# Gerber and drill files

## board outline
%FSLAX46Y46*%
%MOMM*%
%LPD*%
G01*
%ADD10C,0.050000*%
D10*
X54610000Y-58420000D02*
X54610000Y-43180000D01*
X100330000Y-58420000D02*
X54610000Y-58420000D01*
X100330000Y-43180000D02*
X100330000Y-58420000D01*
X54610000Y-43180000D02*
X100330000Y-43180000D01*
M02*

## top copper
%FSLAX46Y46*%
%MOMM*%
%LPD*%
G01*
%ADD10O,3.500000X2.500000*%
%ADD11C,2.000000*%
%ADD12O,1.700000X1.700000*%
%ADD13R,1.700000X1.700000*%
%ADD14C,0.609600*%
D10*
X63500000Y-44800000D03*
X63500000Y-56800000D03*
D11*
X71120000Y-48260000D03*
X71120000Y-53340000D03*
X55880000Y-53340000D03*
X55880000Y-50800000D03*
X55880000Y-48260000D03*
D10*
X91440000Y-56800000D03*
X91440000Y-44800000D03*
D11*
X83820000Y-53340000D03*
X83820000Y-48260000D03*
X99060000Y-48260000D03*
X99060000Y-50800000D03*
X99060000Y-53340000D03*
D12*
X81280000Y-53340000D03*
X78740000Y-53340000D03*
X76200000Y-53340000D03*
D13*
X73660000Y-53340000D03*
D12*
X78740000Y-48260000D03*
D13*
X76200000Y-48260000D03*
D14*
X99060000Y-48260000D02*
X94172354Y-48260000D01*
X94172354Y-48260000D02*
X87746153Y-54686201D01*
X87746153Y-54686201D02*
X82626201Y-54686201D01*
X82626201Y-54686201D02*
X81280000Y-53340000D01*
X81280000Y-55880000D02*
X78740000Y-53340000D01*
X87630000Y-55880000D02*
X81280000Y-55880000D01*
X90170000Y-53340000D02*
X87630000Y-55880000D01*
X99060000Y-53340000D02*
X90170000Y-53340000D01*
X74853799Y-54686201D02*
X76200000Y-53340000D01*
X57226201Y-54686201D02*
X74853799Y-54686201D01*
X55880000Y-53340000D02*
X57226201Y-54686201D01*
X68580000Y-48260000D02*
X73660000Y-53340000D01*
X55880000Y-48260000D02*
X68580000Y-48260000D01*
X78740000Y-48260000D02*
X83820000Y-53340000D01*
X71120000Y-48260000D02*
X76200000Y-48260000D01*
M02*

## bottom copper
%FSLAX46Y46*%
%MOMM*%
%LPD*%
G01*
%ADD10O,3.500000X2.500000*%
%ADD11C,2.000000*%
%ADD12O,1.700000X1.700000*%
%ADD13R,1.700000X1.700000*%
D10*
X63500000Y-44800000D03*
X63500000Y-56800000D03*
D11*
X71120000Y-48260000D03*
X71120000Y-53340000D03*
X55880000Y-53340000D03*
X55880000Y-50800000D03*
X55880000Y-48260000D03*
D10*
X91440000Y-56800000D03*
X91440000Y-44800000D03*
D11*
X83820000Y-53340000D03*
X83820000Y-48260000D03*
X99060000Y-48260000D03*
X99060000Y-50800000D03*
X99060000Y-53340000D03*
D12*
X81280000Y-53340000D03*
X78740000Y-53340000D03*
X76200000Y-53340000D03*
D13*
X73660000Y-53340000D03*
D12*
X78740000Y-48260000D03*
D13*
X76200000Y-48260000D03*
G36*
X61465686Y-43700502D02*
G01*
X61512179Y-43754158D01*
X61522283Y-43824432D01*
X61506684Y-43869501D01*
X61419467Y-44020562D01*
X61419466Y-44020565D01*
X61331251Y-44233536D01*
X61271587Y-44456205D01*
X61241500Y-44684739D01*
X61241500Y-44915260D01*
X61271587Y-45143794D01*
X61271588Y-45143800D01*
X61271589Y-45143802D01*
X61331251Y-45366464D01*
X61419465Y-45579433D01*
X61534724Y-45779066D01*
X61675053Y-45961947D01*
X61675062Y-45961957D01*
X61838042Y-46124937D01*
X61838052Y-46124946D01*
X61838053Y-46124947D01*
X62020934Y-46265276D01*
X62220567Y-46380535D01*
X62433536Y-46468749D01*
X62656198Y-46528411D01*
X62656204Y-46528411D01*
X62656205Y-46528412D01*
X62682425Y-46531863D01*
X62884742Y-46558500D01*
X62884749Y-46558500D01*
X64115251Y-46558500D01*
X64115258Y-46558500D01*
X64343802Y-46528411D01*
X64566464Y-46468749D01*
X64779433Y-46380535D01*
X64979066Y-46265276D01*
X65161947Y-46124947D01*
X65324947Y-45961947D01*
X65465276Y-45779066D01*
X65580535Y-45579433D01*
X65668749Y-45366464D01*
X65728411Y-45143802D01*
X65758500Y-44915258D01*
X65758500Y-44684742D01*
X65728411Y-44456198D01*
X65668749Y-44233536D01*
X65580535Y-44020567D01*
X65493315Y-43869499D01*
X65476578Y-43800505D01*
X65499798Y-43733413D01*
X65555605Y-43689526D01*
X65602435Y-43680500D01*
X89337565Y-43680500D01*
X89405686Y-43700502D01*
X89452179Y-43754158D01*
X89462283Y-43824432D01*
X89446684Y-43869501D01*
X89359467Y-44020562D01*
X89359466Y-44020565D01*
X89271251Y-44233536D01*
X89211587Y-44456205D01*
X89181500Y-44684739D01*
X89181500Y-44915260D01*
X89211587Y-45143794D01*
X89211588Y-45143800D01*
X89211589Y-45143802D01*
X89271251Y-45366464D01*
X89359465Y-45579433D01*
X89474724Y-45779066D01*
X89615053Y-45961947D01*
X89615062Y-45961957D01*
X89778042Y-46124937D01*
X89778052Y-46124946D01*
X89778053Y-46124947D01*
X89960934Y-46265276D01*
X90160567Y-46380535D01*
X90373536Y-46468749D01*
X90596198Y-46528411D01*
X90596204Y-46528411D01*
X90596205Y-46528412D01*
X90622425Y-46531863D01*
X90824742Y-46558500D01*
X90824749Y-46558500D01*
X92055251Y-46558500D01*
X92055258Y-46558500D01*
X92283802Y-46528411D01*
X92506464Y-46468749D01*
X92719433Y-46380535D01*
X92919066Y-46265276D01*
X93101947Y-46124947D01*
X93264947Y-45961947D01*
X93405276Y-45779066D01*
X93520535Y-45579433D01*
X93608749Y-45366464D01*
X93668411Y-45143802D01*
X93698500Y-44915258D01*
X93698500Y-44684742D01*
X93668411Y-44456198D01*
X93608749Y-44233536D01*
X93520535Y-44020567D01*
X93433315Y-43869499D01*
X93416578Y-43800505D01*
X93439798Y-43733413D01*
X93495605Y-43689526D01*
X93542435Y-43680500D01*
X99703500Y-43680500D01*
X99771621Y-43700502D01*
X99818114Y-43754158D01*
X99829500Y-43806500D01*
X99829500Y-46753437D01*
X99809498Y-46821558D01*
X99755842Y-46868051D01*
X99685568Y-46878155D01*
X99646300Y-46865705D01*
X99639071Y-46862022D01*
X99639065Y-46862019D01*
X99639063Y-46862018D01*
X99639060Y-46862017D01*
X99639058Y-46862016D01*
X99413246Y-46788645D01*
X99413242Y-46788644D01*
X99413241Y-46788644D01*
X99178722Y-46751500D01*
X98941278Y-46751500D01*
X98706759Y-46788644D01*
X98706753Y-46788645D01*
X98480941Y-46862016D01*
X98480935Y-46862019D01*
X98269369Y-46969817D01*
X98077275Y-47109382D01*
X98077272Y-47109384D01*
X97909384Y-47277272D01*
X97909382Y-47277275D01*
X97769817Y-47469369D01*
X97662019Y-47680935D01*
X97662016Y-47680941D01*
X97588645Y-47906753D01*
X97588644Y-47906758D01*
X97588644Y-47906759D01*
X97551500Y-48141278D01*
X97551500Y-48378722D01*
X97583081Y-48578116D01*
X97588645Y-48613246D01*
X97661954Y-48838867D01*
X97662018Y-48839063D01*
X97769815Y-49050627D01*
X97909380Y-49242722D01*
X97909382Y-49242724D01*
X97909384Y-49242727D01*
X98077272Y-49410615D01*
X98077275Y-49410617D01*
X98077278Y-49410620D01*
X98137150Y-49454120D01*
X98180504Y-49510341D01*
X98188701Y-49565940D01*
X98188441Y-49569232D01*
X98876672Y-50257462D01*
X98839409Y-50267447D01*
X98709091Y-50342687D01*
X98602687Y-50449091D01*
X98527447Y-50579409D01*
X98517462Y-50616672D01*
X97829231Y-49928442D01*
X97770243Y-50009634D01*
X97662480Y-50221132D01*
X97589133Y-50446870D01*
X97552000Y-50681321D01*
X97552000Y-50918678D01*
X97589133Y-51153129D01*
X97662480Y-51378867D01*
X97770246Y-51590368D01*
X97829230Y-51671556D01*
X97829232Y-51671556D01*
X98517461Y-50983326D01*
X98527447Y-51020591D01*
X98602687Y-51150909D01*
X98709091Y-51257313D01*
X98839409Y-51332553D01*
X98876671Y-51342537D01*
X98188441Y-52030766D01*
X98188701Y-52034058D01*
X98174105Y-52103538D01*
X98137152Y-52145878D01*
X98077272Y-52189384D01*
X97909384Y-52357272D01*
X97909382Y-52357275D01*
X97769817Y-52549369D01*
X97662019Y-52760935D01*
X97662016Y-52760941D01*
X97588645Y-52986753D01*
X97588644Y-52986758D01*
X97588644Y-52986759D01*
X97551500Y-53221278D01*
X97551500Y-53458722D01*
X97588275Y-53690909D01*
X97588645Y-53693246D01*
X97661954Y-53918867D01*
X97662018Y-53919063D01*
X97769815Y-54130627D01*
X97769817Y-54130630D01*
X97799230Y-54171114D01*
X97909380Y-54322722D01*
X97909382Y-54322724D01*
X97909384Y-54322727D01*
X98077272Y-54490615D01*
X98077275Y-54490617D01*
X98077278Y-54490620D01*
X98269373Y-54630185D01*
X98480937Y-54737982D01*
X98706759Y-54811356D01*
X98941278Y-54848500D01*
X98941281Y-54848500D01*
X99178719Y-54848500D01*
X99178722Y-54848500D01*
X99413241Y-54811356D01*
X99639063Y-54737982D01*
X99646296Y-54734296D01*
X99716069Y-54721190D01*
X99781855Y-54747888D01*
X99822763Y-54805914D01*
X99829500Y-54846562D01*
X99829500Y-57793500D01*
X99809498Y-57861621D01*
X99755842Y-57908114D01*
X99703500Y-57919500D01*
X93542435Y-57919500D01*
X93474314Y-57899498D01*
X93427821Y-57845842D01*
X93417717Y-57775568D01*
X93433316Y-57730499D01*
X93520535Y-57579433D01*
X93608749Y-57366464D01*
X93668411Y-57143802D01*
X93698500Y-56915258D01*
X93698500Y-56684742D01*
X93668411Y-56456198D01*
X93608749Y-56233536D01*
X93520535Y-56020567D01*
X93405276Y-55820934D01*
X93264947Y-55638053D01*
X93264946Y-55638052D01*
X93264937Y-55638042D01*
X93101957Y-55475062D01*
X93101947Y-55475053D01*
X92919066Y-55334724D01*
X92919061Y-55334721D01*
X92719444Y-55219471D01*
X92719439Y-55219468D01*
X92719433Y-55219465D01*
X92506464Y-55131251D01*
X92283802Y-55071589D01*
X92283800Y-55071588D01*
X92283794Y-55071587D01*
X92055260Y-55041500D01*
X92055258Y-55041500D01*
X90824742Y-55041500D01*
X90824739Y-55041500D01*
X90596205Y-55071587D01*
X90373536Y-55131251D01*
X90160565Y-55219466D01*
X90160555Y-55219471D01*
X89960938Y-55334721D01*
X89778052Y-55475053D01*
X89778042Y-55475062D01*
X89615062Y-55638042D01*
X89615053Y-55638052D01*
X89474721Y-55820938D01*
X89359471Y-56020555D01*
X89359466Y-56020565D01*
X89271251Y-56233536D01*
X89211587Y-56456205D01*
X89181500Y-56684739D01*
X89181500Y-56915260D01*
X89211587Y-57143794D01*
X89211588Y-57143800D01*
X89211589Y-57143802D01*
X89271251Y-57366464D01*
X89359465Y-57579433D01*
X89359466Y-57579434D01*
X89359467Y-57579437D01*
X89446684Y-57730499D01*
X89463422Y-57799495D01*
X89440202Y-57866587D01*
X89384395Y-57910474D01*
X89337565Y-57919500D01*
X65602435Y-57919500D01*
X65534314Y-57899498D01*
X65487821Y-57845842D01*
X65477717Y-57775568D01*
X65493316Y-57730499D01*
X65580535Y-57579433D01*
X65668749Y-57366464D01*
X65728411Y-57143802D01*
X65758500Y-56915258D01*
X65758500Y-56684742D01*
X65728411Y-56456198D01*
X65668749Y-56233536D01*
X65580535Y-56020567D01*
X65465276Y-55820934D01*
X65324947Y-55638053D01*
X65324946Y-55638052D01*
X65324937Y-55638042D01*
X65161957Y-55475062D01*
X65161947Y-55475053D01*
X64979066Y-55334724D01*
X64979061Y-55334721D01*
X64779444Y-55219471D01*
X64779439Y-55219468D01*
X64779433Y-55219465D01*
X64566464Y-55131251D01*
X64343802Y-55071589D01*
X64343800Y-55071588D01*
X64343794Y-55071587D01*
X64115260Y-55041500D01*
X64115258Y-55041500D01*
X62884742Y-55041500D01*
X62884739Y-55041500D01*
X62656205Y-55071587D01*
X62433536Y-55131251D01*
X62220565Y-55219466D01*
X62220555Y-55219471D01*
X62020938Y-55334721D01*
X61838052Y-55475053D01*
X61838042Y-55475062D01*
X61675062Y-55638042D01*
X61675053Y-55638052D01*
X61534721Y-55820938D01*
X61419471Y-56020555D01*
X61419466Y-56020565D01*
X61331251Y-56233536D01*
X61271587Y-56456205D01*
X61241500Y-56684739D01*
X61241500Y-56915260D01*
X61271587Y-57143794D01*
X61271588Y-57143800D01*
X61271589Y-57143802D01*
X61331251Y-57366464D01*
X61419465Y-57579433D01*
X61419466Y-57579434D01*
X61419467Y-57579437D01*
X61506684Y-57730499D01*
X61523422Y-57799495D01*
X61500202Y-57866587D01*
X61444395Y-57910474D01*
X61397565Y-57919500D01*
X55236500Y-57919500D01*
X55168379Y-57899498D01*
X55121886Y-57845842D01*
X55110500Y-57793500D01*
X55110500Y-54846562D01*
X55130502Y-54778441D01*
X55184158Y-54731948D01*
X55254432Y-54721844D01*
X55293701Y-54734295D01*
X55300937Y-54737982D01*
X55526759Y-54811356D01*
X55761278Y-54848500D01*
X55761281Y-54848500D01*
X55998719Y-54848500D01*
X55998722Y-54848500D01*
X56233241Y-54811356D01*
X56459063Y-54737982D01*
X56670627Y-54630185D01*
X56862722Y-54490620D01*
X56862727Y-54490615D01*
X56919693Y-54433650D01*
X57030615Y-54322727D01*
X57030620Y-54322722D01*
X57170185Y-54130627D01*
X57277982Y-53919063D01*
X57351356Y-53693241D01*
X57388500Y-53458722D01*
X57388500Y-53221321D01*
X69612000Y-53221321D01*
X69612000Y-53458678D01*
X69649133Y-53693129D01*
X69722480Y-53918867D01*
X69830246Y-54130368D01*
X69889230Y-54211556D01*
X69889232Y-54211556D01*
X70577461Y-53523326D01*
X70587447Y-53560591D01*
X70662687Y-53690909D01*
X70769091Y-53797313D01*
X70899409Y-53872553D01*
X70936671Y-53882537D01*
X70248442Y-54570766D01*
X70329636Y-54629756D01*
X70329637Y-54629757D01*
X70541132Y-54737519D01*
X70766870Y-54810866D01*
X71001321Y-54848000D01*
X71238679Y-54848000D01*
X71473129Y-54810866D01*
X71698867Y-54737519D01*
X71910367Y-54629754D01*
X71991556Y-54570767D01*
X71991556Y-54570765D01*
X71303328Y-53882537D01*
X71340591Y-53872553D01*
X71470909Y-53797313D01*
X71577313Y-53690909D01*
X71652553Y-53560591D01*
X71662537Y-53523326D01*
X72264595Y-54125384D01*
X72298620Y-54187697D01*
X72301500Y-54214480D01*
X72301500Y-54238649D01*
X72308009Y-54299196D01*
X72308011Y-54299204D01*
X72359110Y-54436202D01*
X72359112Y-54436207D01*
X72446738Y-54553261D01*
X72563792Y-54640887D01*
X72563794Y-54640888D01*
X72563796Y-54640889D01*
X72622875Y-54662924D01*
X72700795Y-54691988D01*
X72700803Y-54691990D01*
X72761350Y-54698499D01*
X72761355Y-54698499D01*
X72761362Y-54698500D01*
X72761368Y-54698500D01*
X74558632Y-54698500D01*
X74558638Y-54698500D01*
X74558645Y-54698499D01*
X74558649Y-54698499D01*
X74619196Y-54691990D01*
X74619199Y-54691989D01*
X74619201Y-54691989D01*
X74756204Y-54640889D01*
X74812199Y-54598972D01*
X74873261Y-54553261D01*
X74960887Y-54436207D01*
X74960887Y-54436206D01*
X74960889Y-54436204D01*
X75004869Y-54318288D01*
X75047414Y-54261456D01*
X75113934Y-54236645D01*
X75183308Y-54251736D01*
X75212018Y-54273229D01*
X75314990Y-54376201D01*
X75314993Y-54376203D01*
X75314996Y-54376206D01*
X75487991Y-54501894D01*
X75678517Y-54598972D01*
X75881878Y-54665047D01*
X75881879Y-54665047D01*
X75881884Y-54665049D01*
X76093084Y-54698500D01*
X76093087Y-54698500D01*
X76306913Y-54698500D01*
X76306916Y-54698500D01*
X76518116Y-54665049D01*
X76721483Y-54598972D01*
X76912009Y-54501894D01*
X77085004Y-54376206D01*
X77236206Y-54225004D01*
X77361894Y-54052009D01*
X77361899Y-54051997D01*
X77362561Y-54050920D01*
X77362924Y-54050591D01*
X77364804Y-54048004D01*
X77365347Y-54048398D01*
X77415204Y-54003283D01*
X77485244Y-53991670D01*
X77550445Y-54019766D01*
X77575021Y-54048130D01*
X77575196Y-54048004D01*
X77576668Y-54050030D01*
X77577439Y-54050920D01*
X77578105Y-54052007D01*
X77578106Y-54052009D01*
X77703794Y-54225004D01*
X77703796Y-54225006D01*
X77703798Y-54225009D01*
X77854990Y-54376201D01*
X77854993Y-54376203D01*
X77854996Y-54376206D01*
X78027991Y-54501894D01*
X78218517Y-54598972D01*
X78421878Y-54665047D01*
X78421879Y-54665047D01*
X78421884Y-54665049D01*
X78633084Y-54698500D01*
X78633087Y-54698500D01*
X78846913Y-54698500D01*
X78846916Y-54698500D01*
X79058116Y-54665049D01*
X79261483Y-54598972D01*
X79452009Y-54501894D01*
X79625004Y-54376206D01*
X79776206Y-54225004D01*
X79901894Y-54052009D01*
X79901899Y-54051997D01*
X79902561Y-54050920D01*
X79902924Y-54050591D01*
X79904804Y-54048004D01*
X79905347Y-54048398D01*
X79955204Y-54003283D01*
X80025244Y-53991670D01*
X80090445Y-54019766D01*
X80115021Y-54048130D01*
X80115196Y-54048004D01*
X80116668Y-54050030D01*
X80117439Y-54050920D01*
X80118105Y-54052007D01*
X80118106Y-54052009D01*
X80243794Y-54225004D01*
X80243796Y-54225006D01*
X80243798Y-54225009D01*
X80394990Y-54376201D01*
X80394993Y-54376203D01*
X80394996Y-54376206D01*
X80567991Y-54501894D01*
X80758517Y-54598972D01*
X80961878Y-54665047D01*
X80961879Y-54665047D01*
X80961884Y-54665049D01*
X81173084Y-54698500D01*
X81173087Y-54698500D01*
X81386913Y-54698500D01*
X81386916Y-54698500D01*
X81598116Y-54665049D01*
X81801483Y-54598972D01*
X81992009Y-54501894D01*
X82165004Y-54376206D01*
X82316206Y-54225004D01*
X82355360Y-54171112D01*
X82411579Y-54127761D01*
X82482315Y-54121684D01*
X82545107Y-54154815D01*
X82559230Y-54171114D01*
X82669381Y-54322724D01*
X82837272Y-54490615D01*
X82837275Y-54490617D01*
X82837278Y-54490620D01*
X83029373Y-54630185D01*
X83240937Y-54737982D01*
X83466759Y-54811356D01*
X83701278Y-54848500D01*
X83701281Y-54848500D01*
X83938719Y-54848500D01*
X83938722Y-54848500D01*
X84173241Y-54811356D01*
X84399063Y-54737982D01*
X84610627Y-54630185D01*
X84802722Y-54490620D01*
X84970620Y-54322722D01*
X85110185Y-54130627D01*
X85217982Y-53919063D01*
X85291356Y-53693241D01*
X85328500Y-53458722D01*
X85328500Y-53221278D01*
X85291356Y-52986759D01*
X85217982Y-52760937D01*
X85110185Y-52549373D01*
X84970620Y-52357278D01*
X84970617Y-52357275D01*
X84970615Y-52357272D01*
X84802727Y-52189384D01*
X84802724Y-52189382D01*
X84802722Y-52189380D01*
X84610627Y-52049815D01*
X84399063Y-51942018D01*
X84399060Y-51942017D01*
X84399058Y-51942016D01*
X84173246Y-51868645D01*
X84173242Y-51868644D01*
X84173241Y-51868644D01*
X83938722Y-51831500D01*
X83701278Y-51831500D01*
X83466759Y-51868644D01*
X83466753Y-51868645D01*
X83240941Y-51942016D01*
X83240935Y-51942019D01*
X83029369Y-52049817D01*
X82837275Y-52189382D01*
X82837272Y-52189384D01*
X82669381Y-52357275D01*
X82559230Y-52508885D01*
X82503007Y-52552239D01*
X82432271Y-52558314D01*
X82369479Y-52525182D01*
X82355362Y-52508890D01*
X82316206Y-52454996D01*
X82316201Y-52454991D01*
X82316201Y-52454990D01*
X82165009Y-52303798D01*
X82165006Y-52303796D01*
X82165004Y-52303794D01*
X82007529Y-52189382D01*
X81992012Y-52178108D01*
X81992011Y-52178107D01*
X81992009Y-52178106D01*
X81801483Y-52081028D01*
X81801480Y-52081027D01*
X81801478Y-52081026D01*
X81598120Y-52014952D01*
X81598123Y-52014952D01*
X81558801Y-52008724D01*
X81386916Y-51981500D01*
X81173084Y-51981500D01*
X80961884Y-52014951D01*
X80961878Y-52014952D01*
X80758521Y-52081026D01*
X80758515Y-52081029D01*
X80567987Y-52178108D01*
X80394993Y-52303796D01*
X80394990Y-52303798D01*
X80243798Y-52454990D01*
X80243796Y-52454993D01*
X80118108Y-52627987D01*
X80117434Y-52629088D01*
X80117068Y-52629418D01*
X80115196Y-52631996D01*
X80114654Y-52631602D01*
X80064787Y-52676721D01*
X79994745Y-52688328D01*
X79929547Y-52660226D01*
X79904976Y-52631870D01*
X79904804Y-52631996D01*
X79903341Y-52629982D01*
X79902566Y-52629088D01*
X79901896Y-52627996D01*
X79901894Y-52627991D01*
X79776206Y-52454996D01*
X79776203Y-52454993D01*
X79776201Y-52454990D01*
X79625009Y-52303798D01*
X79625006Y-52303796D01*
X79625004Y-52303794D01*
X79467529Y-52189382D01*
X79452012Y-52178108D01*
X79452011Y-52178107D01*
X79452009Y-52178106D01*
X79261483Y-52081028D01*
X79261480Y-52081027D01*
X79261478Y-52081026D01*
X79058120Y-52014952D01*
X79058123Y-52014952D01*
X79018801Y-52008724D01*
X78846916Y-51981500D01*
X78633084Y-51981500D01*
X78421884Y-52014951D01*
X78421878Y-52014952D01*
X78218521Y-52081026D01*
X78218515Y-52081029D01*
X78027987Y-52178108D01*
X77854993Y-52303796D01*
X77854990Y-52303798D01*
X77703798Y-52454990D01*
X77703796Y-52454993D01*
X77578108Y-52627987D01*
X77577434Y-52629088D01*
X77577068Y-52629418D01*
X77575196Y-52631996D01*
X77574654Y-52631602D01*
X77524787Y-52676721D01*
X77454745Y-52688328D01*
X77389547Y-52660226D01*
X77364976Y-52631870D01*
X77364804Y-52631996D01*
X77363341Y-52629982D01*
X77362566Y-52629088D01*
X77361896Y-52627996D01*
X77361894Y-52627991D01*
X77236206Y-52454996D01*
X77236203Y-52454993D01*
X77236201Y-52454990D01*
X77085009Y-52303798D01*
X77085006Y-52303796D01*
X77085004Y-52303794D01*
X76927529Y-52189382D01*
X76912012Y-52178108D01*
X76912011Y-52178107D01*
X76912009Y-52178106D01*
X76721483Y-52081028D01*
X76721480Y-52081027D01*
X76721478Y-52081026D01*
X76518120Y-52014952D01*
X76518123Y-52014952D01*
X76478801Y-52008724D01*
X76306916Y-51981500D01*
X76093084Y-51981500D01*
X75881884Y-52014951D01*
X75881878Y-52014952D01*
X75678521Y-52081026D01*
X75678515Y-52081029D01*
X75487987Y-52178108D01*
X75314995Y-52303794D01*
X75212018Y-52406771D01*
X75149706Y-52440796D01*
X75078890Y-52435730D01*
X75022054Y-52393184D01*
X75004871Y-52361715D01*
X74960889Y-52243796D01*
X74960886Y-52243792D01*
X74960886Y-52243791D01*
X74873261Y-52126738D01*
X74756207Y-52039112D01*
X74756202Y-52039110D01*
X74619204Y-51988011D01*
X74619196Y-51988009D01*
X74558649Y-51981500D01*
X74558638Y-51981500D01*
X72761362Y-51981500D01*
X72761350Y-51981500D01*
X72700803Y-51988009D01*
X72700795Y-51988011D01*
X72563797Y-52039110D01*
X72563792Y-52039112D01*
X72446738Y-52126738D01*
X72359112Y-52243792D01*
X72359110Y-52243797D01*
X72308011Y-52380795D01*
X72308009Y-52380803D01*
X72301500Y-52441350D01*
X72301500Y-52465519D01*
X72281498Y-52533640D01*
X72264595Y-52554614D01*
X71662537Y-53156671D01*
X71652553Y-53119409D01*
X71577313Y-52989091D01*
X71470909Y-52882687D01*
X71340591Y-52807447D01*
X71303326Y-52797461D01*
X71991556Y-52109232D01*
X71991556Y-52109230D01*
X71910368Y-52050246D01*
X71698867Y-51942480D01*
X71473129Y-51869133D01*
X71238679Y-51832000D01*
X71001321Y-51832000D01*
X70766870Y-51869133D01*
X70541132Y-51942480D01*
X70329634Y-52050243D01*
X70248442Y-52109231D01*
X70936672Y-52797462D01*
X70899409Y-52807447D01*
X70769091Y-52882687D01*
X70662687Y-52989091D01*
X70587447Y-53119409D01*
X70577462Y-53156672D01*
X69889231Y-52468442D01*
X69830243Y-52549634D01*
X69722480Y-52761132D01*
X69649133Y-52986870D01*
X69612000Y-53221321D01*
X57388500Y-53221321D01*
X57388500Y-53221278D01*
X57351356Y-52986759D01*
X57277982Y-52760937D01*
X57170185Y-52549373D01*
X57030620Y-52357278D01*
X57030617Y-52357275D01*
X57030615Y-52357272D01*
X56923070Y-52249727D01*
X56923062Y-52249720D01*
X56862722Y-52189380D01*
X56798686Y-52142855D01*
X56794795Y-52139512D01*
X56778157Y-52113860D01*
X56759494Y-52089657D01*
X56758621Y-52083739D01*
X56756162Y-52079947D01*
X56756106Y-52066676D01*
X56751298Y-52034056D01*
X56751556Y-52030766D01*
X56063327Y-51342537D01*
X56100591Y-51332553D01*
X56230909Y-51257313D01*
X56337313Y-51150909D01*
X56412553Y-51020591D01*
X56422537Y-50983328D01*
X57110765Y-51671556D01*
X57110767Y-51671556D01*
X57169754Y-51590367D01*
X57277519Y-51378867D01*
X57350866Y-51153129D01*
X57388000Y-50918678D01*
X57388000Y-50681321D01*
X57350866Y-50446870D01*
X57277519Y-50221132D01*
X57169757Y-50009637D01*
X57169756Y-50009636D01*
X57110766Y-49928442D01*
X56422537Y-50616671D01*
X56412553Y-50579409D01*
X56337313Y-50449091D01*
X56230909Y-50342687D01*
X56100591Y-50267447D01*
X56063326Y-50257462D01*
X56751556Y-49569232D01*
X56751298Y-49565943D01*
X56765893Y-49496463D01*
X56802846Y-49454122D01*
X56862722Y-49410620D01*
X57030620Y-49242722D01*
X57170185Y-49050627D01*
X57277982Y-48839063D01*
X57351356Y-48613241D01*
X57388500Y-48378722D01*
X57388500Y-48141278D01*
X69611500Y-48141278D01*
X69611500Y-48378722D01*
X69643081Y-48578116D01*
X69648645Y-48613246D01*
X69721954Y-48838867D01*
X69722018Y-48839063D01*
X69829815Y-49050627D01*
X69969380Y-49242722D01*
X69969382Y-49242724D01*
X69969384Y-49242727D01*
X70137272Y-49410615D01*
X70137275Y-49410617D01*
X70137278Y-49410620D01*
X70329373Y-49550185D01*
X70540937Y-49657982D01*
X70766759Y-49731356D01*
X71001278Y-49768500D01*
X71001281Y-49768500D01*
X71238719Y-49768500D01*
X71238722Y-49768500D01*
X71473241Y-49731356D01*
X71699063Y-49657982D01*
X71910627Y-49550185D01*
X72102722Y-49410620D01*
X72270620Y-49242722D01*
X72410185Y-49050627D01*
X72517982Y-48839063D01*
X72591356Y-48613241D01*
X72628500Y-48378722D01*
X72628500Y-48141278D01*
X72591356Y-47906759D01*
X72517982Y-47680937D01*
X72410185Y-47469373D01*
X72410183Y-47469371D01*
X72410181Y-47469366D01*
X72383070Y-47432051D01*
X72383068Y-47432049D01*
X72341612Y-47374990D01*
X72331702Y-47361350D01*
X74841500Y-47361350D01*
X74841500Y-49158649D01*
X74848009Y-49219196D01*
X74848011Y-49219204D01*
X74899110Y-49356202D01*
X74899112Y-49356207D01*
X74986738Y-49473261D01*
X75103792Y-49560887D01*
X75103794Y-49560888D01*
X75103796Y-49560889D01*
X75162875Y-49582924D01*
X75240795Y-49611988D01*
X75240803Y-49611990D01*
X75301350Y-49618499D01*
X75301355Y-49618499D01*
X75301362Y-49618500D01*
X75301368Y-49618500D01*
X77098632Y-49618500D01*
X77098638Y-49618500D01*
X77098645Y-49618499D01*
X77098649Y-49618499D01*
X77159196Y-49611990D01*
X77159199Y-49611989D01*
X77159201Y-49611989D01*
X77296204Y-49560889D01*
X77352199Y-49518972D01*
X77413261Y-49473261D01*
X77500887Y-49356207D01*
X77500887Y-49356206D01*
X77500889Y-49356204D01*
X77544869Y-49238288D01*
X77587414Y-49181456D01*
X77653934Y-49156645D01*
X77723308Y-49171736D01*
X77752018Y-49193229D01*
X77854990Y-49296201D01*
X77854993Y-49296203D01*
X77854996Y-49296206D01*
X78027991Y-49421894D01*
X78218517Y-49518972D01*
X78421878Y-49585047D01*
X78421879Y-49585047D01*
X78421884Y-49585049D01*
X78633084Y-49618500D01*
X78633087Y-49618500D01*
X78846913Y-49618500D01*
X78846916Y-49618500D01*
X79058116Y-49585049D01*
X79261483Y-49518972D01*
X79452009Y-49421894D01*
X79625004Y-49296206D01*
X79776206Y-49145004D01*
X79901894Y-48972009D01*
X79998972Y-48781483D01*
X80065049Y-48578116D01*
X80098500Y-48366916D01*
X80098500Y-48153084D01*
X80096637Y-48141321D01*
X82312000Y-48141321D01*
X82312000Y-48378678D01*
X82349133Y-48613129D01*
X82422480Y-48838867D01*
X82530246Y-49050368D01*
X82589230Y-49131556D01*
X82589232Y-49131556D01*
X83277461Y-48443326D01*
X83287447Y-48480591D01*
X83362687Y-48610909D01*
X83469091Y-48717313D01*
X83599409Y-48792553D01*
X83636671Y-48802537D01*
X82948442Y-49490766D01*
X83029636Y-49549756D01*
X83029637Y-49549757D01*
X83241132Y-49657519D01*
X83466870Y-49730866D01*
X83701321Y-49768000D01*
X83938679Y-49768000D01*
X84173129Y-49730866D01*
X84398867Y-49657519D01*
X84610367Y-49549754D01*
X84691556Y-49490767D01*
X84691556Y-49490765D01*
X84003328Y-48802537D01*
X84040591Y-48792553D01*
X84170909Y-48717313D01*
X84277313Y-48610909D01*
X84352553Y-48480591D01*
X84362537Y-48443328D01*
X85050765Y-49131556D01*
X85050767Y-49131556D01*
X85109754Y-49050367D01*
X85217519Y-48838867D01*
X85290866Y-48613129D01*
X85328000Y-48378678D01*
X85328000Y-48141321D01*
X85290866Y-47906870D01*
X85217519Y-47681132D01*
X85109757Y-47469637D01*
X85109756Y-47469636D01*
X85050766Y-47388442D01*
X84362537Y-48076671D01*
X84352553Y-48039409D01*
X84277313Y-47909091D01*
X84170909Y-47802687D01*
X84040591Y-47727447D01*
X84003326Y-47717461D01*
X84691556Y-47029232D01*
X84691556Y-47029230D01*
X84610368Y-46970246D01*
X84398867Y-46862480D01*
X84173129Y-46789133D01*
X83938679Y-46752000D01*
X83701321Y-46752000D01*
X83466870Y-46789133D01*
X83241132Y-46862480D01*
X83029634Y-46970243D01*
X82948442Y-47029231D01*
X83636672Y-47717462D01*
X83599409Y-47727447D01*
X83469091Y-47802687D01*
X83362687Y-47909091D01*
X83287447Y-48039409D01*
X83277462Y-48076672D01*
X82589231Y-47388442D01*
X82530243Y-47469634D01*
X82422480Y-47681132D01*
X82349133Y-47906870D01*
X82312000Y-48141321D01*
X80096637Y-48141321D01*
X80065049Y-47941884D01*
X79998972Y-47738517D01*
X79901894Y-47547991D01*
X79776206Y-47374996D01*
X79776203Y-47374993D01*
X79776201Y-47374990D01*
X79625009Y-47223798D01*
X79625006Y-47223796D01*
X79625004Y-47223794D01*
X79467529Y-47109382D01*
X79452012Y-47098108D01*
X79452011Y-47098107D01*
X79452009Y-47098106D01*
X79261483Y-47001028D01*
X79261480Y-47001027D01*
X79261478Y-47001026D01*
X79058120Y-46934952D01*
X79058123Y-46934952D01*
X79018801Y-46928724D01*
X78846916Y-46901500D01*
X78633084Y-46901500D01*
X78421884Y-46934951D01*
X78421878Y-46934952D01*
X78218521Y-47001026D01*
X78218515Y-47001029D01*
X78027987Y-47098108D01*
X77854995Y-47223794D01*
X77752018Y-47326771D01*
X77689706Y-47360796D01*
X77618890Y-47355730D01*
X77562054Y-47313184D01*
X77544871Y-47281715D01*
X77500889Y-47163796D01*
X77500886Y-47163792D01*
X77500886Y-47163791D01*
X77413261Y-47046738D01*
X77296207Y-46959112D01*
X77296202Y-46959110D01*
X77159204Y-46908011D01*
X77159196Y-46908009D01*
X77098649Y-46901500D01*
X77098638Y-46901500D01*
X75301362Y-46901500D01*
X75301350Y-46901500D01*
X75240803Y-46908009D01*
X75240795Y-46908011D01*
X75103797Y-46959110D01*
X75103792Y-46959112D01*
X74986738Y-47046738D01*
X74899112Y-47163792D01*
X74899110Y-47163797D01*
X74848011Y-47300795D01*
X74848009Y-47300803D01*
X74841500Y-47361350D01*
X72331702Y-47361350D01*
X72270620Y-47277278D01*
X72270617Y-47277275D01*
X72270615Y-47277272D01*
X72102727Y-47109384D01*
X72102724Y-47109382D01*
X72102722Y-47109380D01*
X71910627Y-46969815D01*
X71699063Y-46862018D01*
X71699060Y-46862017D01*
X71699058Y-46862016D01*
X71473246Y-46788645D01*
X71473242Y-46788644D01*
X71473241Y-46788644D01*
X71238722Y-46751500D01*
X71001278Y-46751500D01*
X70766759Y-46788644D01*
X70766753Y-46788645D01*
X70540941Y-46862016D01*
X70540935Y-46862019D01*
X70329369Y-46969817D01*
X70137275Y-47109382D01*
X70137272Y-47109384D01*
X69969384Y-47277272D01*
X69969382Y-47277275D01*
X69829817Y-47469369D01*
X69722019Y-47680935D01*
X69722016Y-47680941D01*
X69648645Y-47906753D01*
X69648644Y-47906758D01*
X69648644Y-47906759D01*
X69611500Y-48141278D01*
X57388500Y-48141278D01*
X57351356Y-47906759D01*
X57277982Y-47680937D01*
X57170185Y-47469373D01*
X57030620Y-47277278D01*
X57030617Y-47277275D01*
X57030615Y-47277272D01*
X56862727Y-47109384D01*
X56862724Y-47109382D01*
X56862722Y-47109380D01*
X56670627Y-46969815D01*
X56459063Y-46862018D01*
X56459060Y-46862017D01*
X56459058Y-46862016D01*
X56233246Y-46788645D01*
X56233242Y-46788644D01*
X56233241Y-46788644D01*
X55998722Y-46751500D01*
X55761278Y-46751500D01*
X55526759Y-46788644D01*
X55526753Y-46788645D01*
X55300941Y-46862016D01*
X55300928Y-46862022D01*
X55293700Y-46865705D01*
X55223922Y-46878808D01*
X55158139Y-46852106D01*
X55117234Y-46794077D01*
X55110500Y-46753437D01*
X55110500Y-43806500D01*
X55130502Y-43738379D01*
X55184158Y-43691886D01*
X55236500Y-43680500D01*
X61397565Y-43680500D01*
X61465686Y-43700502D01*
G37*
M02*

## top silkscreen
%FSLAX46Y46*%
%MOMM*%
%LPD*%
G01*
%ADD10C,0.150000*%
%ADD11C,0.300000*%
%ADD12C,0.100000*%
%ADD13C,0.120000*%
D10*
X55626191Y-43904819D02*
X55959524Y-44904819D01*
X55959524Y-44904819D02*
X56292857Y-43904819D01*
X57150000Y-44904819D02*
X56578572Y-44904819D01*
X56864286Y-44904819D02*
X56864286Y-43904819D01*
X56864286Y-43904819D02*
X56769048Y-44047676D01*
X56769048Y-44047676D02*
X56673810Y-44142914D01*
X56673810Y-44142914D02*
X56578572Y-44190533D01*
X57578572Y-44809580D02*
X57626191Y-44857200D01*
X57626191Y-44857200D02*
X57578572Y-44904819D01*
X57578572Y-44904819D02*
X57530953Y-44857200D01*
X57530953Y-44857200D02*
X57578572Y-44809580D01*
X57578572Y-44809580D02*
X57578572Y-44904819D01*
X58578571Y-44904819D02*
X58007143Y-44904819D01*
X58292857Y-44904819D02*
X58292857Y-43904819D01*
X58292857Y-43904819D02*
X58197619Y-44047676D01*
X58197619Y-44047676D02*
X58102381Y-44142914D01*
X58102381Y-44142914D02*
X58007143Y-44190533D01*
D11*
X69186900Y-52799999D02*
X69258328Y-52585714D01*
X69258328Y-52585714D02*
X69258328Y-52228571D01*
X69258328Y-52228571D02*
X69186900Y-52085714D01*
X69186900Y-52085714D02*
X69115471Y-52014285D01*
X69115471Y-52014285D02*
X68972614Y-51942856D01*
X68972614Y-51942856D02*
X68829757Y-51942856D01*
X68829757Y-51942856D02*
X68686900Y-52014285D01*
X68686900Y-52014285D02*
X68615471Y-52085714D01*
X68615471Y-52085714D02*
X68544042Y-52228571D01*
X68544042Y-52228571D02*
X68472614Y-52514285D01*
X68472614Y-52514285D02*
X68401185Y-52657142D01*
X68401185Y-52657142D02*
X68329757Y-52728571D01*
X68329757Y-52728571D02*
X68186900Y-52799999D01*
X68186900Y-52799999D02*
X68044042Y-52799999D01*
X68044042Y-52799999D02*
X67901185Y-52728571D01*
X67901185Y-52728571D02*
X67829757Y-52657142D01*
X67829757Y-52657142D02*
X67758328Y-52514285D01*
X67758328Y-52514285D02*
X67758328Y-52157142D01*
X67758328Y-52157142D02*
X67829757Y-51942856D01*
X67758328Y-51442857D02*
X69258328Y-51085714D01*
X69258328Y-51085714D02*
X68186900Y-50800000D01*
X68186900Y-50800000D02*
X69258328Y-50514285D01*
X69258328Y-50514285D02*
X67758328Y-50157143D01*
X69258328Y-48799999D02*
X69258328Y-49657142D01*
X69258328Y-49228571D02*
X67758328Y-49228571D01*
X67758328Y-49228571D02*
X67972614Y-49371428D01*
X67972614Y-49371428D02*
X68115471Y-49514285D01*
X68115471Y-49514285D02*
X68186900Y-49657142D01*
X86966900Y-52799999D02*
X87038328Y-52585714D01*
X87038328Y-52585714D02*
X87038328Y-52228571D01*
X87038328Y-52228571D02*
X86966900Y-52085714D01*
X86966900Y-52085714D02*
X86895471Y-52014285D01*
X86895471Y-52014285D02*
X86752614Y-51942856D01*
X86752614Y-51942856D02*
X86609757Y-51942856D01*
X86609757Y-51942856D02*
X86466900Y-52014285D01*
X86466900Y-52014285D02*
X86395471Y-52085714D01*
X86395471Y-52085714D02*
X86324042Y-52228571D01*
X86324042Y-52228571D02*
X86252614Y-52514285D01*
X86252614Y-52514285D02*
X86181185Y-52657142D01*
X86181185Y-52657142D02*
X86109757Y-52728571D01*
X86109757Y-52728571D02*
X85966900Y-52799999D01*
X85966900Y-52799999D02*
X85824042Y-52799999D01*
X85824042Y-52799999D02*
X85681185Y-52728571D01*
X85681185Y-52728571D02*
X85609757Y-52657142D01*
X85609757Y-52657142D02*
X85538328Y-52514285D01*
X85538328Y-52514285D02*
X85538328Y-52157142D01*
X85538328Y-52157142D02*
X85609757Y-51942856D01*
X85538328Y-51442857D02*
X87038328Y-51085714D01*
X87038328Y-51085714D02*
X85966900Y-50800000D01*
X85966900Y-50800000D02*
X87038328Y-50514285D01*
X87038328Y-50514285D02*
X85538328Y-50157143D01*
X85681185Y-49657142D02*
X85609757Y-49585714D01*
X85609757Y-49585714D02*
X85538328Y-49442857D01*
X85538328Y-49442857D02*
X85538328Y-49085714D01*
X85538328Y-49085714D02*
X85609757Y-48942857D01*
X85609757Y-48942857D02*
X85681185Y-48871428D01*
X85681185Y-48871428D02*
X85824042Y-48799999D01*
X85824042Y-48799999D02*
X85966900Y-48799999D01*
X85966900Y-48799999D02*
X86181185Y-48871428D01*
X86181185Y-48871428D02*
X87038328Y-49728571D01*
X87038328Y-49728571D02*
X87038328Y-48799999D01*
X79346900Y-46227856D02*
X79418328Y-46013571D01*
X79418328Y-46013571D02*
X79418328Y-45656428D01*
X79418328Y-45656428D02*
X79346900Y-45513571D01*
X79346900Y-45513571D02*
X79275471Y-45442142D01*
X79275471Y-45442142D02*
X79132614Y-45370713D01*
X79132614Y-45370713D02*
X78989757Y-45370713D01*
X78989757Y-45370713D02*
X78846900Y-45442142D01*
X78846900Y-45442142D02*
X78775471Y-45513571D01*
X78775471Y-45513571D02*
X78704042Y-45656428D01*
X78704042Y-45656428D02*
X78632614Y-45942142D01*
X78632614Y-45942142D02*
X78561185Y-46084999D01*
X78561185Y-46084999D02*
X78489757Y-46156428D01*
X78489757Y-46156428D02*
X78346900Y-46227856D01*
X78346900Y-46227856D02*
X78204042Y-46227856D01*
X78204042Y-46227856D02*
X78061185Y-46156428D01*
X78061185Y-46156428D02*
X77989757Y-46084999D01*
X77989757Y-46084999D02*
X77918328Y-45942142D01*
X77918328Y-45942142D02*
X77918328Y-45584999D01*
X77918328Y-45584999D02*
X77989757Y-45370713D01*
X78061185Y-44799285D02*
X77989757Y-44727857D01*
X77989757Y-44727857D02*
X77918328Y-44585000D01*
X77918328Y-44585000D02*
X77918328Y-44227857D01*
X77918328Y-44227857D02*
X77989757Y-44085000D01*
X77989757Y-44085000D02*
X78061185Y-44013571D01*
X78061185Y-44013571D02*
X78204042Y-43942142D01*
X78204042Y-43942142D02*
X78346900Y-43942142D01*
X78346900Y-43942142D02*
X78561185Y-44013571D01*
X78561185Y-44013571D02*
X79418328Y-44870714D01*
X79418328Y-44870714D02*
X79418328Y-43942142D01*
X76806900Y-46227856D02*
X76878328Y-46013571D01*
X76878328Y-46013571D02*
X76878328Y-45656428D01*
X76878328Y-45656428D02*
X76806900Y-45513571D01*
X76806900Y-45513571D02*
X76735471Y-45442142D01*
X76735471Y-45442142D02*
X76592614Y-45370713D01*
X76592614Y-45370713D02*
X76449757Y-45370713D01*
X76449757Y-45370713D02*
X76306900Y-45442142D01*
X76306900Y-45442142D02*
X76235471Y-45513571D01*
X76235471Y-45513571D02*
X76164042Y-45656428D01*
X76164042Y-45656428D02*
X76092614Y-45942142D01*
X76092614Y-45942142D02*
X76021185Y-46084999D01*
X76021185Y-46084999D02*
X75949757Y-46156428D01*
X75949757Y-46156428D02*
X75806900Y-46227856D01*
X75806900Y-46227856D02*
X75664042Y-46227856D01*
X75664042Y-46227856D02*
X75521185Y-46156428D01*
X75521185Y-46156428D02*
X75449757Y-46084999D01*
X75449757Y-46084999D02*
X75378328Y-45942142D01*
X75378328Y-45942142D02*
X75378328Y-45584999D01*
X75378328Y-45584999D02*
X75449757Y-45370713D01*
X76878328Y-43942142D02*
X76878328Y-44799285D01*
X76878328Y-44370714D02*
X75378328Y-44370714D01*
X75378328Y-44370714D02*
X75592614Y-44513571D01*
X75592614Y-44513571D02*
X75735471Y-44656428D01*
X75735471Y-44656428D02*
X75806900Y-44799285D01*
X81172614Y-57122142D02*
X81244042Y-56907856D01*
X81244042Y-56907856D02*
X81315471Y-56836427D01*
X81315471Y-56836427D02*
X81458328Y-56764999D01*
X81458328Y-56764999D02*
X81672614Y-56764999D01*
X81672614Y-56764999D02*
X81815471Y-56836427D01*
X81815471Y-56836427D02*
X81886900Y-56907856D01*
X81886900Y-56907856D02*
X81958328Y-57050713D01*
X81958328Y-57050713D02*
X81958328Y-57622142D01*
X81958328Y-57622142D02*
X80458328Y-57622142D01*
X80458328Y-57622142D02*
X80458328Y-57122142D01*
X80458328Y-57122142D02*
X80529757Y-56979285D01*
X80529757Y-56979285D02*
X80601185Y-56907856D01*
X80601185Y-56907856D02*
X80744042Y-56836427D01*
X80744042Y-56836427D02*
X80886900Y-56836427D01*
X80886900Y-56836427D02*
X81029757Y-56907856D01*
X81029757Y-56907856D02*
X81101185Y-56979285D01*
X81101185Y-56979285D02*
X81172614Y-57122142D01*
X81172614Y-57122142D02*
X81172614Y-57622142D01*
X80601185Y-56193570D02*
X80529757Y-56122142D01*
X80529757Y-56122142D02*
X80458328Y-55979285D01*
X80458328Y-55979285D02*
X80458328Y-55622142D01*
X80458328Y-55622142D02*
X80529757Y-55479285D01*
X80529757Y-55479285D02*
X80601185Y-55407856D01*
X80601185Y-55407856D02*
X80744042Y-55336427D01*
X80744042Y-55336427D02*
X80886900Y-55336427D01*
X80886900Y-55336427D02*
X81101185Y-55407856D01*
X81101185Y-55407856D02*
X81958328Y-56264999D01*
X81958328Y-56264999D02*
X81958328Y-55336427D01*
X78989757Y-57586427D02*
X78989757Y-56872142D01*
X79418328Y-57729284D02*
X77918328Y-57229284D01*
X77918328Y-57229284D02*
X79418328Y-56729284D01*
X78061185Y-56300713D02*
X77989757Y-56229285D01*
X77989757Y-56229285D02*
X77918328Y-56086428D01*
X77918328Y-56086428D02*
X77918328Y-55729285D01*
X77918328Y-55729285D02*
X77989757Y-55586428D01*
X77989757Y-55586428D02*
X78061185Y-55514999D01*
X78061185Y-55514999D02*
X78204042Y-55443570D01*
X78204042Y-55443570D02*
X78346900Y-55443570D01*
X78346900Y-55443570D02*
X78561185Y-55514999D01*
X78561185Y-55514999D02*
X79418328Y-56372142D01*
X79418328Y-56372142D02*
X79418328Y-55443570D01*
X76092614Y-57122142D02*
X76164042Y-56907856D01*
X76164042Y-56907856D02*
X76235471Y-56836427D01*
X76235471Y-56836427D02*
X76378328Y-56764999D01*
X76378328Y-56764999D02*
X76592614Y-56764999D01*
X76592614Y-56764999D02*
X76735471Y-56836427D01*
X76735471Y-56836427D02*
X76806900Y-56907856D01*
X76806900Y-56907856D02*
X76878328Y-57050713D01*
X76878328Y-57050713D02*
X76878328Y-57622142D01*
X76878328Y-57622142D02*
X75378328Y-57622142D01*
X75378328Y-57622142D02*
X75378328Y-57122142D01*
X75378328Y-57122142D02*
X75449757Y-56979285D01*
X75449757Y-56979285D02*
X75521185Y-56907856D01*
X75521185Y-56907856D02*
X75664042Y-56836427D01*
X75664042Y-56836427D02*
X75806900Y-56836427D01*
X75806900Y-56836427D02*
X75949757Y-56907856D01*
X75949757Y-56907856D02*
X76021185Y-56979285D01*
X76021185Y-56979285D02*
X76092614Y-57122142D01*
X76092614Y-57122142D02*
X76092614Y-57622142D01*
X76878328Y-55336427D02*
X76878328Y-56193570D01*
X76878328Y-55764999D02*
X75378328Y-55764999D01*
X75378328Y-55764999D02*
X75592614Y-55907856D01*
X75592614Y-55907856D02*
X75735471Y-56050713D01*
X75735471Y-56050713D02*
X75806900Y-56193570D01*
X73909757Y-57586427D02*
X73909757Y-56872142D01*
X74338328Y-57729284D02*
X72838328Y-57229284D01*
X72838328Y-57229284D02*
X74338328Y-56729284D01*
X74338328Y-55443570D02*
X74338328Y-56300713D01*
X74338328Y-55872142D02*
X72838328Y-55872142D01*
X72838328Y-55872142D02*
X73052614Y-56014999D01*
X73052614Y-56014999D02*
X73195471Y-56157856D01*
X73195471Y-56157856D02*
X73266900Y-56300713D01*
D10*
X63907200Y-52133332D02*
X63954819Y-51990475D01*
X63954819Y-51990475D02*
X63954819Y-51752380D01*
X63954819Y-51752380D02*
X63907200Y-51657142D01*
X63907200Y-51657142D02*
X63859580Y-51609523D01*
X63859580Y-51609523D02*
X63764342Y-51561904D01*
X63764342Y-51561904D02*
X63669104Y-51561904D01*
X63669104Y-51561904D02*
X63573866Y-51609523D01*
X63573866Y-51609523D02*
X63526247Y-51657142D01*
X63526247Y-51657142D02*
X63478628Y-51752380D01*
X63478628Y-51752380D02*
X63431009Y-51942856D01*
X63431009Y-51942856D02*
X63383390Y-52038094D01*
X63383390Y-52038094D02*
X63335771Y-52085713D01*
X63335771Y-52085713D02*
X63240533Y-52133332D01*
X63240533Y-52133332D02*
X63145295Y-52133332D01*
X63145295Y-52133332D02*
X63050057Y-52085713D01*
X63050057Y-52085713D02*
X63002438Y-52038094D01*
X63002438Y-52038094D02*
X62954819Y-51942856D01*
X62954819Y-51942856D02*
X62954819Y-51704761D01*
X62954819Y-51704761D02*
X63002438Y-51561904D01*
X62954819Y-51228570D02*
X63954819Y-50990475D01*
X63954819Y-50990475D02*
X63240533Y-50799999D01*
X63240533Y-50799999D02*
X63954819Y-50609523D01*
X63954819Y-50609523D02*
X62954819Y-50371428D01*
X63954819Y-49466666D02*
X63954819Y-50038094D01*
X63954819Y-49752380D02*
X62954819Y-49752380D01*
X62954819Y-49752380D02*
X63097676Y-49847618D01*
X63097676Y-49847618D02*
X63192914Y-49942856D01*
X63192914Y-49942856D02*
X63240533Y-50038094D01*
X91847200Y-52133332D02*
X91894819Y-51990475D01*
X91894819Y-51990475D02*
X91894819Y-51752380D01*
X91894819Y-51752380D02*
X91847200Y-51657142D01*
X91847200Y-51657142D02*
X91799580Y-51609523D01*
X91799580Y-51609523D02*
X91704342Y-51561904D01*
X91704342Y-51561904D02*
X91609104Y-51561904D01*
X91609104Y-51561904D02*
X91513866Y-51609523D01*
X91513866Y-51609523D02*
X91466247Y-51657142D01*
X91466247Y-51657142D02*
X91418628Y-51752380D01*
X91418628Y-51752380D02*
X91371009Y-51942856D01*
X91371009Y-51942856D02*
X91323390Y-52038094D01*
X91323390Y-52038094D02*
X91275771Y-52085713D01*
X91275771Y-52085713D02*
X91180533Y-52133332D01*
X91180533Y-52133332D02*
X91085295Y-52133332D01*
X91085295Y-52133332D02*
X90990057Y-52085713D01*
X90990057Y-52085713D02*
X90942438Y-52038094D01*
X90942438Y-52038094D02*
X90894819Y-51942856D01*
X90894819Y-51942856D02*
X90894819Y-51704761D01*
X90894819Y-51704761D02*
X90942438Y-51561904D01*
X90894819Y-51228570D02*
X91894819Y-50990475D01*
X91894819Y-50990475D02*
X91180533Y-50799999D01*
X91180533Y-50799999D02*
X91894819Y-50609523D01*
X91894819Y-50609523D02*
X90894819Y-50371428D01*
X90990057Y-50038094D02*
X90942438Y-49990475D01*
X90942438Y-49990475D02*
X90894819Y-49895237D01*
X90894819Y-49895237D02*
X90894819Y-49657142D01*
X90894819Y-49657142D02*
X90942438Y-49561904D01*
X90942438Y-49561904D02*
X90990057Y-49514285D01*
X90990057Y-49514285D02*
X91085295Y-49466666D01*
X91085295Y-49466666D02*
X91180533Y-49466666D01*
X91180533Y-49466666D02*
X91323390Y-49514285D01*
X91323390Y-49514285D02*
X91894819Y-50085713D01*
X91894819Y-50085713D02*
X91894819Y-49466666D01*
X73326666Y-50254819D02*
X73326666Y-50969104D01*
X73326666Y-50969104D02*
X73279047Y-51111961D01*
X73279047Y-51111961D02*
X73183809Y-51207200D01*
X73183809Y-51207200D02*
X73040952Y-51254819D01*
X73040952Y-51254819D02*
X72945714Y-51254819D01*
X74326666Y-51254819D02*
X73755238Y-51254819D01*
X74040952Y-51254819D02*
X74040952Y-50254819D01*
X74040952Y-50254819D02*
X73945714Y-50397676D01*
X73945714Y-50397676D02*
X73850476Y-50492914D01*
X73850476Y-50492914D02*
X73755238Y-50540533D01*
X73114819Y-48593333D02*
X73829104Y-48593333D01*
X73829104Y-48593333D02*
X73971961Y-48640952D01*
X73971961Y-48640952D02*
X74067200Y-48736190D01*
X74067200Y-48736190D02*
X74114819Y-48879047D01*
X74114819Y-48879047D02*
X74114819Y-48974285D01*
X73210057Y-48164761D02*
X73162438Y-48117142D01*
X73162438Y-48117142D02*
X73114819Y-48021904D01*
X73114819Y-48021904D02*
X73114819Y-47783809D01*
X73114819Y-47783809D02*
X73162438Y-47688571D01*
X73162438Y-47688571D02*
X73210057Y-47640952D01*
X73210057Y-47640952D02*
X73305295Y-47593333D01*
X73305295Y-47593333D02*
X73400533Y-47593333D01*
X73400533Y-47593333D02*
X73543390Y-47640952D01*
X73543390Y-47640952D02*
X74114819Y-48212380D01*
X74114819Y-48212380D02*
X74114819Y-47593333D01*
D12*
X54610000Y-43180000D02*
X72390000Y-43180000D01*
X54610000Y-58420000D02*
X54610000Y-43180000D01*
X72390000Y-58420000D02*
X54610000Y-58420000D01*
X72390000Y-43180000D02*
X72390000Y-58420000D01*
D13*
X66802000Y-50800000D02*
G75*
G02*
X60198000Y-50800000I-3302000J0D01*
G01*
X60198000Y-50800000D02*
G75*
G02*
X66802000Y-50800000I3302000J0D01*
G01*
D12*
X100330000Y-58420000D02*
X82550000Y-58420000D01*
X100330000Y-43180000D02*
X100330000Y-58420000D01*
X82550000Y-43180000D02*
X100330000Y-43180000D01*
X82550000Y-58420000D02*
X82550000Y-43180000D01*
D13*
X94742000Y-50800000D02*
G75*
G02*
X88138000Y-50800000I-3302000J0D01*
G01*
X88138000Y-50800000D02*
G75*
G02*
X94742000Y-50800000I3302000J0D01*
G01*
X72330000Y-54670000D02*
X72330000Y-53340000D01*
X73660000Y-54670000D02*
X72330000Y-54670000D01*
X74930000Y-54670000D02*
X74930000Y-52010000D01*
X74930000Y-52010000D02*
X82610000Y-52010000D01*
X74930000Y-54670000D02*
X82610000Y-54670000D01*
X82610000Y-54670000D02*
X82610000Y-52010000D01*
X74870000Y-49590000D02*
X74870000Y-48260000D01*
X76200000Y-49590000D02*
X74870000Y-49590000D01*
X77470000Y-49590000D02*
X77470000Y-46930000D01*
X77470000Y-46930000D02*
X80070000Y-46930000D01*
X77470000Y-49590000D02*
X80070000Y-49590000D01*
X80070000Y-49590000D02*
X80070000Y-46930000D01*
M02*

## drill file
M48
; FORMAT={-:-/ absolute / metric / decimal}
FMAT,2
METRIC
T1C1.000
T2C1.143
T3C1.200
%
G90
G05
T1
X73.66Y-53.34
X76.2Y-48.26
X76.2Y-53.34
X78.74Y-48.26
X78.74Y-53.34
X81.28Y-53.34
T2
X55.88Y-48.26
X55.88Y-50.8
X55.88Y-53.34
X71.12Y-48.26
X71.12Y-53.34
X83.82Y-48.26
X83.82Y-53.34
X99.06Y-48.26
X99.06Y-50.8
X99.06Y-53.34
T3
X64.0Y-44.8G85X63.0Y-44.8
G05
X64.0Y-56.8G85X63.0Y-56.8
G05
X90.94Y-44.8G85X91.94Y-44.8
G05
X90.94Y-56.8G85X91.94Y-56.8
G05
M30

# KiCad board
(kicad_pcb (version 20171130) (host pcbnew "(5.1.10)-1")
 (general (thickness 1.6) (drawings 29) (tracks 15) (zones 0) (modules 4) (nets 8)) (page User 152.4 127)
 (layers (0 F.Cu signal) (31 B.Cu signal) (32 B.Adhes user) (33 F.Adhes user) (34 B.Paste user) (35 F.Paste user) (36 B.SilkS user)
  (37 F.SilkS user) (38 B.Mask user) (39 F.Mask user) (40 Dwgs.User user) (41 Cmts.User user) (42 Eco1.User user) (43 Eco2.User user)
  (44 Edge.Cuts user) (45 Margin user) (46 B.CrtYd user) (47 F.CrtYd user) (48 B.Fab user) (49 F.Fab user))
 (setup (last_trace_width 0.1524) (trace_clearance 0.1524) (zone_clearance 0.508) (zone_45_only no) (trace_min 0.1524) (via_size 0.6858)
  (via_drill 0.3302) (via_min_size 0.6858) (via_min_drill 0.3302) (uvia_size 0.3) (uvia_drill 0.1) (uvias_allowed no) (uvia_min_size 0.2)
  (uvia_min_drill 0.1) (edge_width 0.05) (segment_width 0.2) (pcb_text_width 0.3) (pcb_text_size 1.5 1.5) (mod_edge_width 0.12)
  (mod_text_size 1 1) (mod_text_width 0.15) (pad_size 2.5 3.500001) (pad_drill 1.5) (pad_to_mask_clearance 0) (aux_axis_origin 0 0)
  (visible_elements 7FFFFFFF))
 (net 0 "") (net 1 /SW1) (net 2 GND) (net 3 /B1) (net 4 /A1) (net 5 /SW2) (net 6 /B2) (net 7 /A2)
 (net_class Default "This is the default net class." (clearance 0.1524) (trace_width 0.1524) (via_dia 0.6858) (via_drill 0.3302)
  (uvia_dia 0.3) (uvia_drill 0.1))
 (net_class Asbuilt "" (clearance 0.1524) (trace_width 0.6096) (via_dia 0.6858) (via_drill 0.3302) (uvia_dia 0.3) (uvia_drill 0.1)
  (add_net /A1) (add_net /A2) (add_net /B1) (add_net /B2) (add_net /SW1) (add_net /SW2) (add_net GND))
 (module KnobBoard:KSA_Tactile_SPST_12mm (layer F.Cu) (at 63.5 50.8 270)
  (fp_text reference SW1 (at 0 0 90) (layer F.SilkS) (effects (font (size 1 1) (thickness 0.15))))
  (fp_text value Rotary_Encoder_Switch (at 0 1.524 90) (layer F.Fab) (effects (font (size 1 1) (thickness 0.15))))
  (fp_line (start -7.62 8.89) (end -7.62 -8.89) (layer F.SilkS) (width 0.1))
  (fp_line (start 7.62 8.89) (end -7.62 8.89) (layer F.SilkS) (width 0.1))
  (fp_line (start 7.62 -8.89) (end 7.62 8.89) (layer F.SilkS) (width 0.1))
  (fp_line (start -7.62 -8.89) (end 7.62 -8.89) (layer F.SilkS) (width 0.1))
  (fp_circle (center 0 0) (end 3.302 0) (layer F.SilkS) (width 0.12))
  (pad G thru_hole oval (at -6 0 270) (size 2.5 3.5) (drill oval 1.2 2.2) (layers *.Cu *.Mask))
  (pad G thru_hole oval (at 6 0 270) (size 2.5 3.5) (drill oval 1.2 2.2) (layers *.Cu *.Mask))
  (pad S1 thru_hole circle (at -2.54 -7.62 270) (size 2 2) (drill 1.143) (layers *.Cu *.Mask) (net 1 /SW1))
  (pad S2 thru_hole circle (at 2.54 -7.62 270) (size 2 2) (drill 1.143) (layers *.Cu *.Mask) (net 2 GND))
  (pad B thru_hole circle (at 2.54 7.62 270) (size 2 2) (drill 1.143) (layers *.Cu *.Mask) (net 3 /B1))
  (pad C thru_hole circle (at 0 7.62 270) (size 2 2) (drill 1.143) (layers *.Cu *.Mask) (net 2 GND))
  (pad A thru_hole circle (at -2.54 7.62 270) (size 2 2) (drill 1.143) (layers *.Cu *.Mask) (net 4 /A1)))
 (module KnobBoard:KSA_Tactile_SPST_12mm (layer F.Cu) (at 91.44 50.8 90)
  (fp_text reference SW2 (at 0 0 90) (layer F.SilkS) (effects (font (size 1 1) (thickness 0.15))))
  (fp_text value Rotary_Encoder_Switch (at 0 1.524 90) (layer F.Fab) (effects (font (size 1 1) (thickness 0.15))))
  (fp_line (start -7.62 8.89) (end -7.62 -8.89) (layer F.SilkS) (width 0.1))
  (fp_line (start 7.62 8.89) (end -7.62 8.89) (layer F.SilkS) (width 0.1))
  (fp_line (start 7.62 -8.89) (end 7.62 8.89) (layer F.SilkS) (width 0.1))
  (fp_line (start -7.62 -8.89) (end 7.62 -8.89) (layer F.SilkS) (width 0.1))
  (fp_circle (center 0 0) (end 3.302 0) (layer F.SilkS) (width 0.12))
  (pad G thru_hole oval (at -6 0 90) (size 2.5 3.5) (drill oval 1.2 2.2) (layers *.Cu *.Mask))
  (pad G thru_hole oval (at 6 0 90) (size 2.5 3.5) (drill oval 1.2 2.2) (layers *.Cu *.Mask))
  (pad S1 thru_hole circle (at -2.54 -7.62 90) (size 2 2) (drill 1.143) (layers *.Cu *.Mask) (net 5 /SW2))
  (pad S2 thru_hole circle (at 2.54 -7.62 90) (size 2 2) (drill 1.143) (layers *.Cu *.Mask) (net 2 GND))
  (pad B thru_hole circle (at 2.54 7.62 90) (size 2 2) (drill 1.143) (layers *.Cu *.Mask) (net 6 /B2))
  (pad C thru_hole circle (at 0 7.62 90) (size 2 2) (drill 1.143) (layers *.Cu *.Mask) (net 2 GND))
  (pad A thru_hole circle (at -2.54 7.62 90) (size 2 2) (drill 1.143) (layers *.Cu *.Mask) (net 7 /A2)))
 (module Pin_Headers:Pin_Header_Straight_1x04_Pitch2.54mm (layer F.Cu) (at 73.66 53.34 90)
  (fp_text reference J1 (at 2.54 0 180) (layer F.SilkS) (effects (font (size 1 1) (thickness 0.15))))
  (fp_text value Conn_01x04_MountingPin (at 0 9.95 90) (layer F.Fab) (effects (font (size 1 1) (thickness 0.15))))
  (fp_line (start -1.33 -1.33) (end 0 -1.33) (layer F.SilkS) (width 0.12))
  (fp_line (start -1.33 0) (end -1.33 -1.33) (layer F.SilkS) (width 0.12))
  (fp_line (start -1.33 1.27) (end 1.33 1.27) (layer F.SilkS) (width 0.12))
  (fp_line (start 1.33 1.27) (end 1.33 8.95) (layer F.SilkS) (width 0.12))
  (fp_line (start -1.33 1.27) (end -1.33 8.95) (layer F.SilkS) (width 0.12))
  (fp_line (start -1.33 8.95) (end 1.33 8.95) (layer F.SilkS) (width 0.12))
  (pad 4 thru_hole oval (at 0 7.62 90) (size 1.7 1.7) (drill 1) (layers *.Cu *.Mask) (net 6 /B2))
  (pad 3 thru_hole oval (at 0 5.08 90) (size 1.7 1.7) (drill 1) (layers *.Cu *.Mask) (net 7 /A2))
  (pad 2 thru_hole oval (at 0 2.54 90) (size 1.7 1.7) (drill 1) (layers *.Cu *.Mask) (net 3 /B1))
  (pad 1 thru_hole rect (at 0 0 90) (size 1.7 1.7) (drill 1) (layers *.Cu *.Mask) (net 4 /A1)))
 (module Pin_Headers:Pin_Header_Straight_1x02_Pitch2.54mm (layer F.Cu) (at 76.2 48.26 90)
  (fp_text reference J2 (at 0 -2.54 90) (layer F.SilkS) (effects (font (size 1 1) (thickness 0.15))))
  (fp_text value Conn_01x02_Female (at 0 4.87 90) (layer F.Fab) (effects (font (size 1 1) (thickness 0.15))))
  (fp_line (start -1.33 -1.33) (end 0 -1.33) (layer F.SilkS) (width 0.12))
  (fp_line (start -1.33 0) (end -1.33 -1.33) (layer F.SilkS) (width 0.12))
  (fp_line (start -1.33 1.27) (end 1.33 1.27) (layer F.SilkS) (width 0.12))
  (fp_line (start 1.33 1.27) (end 1.33 3.87) (layer F.SilkS) (width 0.12))
  (fp_line (start -1.33 1.27) (end -1.33 3.87) (layer F.SilkS) (width 0.12))
  (fp_line (start -1.33 3.87) (end 1.33 3.87) (layer F.SilkS) (width 0.12))
  (pad 2 thru_hole oval (at 0 2.54 90) (size 1.7 1.7) (drill 1) (layers *.Cu *.Mask) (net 5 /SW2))
  (pad 1 thru_hole rect (at 0 0 90) (size 1.7 1.7) (drill 1) (layers *.Cu *.Mask) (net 1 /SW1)))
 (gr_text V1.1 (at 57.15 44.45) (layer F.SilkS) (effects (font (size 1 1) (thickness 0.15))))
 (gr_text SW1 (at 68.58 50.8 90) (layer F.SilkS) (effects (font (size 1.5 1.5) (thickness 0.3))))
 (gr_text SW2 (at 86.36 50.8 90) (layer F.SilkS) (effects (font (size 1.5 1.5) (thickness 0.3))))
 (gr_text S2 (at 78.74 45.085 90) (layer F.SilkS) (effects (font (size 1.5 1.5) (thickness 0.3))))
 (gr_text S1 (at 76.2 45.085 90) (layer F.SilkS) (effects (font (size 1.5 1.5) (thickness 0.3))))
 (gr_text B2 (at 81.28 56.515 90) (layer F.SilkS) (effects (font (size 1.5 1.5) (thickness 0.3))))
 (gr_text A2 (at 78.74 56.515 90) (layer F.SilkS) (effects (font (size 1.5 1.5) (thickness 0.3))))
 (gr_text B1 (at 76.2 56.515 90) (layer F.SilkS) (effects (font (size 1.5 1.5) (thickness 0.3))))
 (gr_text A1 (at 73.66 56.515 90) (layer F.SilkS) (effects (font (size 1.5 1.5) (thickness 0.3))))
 (gr_line (start 54.61 58.42) (end 54.61 43.18) (layer Edge.Cuts) (width 0.05))
 (gr_line (start 100.33 58.42) (end 54.61 58.42) (layer Edge.Cuts) (width 0.05))
 (gr_line (start 100.33 43.18) (end 100.33 58.42) (layer Edge.Cuts) (width 0.05))
 (gr_line (start 54.61 43.18) (end 100.33 43.18) (layer Edge.Cuts) (width 0.05))
 (segment (start 99.06 48.26) (end 94.172354 48.26) (width 0.6096) (layer F.Cu) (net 6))
 (segment (start 94.172354 48.26) (end 87.746153 54.686201) (width 0.6096) (layer F.Cu) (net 6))
 (segment (start 87.746153 54.686201) (end 82.626201 54.686201) (width 0.6096) (layer F.Cu) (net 6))
 (segment (start 82.626201 54.686201) (end 81.28 53.34) (width 0.6096) (layer F.Cu) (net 6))
 (segment (start 81.28 55.88) (end 78.74 53.34) (width 0.6096) (layer F.Cu) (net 7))
 (segment (start 87.63 55.88) (end 81.28 55.88) (width 0.6096) (layer F.Cu) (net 7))
 (segment (start 90.17 53.34) (end 87.63 55.88) (width 0.6096) (layer F.Cu) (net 7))
 (segment (start 99.06 53.34) (end 90.17 53.34) (width 0.6096) (layer F.Cu) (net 7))
 (segment (start 74.853799 54.686201) (end 76.2 53.34) (width 0.6096) (layer F.Cu) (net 3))
 (segment (start 57.226201 54.686201) (end 74.853799 54.686201) (width 0.6096) (layer F.Cu) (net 3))
 (segment (start 55.88 53.34) (end 57.226201 54.686201) (width 0.6096) (layer F.Cu) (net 3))
 (segment (start 68.58 48.26) (end 73.66 53.34) (width 0.6096) (layer F.Cu) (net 4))
 (segment (start 55.88 48.26) (end 68.58 48.26) (width 0.6096) (layer F.Cu) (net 4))
 (segment (start 78.74 48.26) (end 83.82 53.34) (width 0.6096) (layer F.Cu) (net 5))
 (segment (start 71.12 48.26) (end 76.2 48.26) (width 0.6096) (layer F.Cu) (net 1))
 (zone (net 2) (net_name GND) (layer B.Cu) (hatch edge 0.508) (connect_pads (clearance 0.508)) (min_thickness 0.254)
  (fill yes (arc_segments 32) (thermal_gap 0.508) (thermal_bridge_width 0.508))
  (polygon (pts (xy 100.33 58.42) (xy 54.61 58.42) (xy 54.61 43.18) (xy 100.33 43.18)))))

